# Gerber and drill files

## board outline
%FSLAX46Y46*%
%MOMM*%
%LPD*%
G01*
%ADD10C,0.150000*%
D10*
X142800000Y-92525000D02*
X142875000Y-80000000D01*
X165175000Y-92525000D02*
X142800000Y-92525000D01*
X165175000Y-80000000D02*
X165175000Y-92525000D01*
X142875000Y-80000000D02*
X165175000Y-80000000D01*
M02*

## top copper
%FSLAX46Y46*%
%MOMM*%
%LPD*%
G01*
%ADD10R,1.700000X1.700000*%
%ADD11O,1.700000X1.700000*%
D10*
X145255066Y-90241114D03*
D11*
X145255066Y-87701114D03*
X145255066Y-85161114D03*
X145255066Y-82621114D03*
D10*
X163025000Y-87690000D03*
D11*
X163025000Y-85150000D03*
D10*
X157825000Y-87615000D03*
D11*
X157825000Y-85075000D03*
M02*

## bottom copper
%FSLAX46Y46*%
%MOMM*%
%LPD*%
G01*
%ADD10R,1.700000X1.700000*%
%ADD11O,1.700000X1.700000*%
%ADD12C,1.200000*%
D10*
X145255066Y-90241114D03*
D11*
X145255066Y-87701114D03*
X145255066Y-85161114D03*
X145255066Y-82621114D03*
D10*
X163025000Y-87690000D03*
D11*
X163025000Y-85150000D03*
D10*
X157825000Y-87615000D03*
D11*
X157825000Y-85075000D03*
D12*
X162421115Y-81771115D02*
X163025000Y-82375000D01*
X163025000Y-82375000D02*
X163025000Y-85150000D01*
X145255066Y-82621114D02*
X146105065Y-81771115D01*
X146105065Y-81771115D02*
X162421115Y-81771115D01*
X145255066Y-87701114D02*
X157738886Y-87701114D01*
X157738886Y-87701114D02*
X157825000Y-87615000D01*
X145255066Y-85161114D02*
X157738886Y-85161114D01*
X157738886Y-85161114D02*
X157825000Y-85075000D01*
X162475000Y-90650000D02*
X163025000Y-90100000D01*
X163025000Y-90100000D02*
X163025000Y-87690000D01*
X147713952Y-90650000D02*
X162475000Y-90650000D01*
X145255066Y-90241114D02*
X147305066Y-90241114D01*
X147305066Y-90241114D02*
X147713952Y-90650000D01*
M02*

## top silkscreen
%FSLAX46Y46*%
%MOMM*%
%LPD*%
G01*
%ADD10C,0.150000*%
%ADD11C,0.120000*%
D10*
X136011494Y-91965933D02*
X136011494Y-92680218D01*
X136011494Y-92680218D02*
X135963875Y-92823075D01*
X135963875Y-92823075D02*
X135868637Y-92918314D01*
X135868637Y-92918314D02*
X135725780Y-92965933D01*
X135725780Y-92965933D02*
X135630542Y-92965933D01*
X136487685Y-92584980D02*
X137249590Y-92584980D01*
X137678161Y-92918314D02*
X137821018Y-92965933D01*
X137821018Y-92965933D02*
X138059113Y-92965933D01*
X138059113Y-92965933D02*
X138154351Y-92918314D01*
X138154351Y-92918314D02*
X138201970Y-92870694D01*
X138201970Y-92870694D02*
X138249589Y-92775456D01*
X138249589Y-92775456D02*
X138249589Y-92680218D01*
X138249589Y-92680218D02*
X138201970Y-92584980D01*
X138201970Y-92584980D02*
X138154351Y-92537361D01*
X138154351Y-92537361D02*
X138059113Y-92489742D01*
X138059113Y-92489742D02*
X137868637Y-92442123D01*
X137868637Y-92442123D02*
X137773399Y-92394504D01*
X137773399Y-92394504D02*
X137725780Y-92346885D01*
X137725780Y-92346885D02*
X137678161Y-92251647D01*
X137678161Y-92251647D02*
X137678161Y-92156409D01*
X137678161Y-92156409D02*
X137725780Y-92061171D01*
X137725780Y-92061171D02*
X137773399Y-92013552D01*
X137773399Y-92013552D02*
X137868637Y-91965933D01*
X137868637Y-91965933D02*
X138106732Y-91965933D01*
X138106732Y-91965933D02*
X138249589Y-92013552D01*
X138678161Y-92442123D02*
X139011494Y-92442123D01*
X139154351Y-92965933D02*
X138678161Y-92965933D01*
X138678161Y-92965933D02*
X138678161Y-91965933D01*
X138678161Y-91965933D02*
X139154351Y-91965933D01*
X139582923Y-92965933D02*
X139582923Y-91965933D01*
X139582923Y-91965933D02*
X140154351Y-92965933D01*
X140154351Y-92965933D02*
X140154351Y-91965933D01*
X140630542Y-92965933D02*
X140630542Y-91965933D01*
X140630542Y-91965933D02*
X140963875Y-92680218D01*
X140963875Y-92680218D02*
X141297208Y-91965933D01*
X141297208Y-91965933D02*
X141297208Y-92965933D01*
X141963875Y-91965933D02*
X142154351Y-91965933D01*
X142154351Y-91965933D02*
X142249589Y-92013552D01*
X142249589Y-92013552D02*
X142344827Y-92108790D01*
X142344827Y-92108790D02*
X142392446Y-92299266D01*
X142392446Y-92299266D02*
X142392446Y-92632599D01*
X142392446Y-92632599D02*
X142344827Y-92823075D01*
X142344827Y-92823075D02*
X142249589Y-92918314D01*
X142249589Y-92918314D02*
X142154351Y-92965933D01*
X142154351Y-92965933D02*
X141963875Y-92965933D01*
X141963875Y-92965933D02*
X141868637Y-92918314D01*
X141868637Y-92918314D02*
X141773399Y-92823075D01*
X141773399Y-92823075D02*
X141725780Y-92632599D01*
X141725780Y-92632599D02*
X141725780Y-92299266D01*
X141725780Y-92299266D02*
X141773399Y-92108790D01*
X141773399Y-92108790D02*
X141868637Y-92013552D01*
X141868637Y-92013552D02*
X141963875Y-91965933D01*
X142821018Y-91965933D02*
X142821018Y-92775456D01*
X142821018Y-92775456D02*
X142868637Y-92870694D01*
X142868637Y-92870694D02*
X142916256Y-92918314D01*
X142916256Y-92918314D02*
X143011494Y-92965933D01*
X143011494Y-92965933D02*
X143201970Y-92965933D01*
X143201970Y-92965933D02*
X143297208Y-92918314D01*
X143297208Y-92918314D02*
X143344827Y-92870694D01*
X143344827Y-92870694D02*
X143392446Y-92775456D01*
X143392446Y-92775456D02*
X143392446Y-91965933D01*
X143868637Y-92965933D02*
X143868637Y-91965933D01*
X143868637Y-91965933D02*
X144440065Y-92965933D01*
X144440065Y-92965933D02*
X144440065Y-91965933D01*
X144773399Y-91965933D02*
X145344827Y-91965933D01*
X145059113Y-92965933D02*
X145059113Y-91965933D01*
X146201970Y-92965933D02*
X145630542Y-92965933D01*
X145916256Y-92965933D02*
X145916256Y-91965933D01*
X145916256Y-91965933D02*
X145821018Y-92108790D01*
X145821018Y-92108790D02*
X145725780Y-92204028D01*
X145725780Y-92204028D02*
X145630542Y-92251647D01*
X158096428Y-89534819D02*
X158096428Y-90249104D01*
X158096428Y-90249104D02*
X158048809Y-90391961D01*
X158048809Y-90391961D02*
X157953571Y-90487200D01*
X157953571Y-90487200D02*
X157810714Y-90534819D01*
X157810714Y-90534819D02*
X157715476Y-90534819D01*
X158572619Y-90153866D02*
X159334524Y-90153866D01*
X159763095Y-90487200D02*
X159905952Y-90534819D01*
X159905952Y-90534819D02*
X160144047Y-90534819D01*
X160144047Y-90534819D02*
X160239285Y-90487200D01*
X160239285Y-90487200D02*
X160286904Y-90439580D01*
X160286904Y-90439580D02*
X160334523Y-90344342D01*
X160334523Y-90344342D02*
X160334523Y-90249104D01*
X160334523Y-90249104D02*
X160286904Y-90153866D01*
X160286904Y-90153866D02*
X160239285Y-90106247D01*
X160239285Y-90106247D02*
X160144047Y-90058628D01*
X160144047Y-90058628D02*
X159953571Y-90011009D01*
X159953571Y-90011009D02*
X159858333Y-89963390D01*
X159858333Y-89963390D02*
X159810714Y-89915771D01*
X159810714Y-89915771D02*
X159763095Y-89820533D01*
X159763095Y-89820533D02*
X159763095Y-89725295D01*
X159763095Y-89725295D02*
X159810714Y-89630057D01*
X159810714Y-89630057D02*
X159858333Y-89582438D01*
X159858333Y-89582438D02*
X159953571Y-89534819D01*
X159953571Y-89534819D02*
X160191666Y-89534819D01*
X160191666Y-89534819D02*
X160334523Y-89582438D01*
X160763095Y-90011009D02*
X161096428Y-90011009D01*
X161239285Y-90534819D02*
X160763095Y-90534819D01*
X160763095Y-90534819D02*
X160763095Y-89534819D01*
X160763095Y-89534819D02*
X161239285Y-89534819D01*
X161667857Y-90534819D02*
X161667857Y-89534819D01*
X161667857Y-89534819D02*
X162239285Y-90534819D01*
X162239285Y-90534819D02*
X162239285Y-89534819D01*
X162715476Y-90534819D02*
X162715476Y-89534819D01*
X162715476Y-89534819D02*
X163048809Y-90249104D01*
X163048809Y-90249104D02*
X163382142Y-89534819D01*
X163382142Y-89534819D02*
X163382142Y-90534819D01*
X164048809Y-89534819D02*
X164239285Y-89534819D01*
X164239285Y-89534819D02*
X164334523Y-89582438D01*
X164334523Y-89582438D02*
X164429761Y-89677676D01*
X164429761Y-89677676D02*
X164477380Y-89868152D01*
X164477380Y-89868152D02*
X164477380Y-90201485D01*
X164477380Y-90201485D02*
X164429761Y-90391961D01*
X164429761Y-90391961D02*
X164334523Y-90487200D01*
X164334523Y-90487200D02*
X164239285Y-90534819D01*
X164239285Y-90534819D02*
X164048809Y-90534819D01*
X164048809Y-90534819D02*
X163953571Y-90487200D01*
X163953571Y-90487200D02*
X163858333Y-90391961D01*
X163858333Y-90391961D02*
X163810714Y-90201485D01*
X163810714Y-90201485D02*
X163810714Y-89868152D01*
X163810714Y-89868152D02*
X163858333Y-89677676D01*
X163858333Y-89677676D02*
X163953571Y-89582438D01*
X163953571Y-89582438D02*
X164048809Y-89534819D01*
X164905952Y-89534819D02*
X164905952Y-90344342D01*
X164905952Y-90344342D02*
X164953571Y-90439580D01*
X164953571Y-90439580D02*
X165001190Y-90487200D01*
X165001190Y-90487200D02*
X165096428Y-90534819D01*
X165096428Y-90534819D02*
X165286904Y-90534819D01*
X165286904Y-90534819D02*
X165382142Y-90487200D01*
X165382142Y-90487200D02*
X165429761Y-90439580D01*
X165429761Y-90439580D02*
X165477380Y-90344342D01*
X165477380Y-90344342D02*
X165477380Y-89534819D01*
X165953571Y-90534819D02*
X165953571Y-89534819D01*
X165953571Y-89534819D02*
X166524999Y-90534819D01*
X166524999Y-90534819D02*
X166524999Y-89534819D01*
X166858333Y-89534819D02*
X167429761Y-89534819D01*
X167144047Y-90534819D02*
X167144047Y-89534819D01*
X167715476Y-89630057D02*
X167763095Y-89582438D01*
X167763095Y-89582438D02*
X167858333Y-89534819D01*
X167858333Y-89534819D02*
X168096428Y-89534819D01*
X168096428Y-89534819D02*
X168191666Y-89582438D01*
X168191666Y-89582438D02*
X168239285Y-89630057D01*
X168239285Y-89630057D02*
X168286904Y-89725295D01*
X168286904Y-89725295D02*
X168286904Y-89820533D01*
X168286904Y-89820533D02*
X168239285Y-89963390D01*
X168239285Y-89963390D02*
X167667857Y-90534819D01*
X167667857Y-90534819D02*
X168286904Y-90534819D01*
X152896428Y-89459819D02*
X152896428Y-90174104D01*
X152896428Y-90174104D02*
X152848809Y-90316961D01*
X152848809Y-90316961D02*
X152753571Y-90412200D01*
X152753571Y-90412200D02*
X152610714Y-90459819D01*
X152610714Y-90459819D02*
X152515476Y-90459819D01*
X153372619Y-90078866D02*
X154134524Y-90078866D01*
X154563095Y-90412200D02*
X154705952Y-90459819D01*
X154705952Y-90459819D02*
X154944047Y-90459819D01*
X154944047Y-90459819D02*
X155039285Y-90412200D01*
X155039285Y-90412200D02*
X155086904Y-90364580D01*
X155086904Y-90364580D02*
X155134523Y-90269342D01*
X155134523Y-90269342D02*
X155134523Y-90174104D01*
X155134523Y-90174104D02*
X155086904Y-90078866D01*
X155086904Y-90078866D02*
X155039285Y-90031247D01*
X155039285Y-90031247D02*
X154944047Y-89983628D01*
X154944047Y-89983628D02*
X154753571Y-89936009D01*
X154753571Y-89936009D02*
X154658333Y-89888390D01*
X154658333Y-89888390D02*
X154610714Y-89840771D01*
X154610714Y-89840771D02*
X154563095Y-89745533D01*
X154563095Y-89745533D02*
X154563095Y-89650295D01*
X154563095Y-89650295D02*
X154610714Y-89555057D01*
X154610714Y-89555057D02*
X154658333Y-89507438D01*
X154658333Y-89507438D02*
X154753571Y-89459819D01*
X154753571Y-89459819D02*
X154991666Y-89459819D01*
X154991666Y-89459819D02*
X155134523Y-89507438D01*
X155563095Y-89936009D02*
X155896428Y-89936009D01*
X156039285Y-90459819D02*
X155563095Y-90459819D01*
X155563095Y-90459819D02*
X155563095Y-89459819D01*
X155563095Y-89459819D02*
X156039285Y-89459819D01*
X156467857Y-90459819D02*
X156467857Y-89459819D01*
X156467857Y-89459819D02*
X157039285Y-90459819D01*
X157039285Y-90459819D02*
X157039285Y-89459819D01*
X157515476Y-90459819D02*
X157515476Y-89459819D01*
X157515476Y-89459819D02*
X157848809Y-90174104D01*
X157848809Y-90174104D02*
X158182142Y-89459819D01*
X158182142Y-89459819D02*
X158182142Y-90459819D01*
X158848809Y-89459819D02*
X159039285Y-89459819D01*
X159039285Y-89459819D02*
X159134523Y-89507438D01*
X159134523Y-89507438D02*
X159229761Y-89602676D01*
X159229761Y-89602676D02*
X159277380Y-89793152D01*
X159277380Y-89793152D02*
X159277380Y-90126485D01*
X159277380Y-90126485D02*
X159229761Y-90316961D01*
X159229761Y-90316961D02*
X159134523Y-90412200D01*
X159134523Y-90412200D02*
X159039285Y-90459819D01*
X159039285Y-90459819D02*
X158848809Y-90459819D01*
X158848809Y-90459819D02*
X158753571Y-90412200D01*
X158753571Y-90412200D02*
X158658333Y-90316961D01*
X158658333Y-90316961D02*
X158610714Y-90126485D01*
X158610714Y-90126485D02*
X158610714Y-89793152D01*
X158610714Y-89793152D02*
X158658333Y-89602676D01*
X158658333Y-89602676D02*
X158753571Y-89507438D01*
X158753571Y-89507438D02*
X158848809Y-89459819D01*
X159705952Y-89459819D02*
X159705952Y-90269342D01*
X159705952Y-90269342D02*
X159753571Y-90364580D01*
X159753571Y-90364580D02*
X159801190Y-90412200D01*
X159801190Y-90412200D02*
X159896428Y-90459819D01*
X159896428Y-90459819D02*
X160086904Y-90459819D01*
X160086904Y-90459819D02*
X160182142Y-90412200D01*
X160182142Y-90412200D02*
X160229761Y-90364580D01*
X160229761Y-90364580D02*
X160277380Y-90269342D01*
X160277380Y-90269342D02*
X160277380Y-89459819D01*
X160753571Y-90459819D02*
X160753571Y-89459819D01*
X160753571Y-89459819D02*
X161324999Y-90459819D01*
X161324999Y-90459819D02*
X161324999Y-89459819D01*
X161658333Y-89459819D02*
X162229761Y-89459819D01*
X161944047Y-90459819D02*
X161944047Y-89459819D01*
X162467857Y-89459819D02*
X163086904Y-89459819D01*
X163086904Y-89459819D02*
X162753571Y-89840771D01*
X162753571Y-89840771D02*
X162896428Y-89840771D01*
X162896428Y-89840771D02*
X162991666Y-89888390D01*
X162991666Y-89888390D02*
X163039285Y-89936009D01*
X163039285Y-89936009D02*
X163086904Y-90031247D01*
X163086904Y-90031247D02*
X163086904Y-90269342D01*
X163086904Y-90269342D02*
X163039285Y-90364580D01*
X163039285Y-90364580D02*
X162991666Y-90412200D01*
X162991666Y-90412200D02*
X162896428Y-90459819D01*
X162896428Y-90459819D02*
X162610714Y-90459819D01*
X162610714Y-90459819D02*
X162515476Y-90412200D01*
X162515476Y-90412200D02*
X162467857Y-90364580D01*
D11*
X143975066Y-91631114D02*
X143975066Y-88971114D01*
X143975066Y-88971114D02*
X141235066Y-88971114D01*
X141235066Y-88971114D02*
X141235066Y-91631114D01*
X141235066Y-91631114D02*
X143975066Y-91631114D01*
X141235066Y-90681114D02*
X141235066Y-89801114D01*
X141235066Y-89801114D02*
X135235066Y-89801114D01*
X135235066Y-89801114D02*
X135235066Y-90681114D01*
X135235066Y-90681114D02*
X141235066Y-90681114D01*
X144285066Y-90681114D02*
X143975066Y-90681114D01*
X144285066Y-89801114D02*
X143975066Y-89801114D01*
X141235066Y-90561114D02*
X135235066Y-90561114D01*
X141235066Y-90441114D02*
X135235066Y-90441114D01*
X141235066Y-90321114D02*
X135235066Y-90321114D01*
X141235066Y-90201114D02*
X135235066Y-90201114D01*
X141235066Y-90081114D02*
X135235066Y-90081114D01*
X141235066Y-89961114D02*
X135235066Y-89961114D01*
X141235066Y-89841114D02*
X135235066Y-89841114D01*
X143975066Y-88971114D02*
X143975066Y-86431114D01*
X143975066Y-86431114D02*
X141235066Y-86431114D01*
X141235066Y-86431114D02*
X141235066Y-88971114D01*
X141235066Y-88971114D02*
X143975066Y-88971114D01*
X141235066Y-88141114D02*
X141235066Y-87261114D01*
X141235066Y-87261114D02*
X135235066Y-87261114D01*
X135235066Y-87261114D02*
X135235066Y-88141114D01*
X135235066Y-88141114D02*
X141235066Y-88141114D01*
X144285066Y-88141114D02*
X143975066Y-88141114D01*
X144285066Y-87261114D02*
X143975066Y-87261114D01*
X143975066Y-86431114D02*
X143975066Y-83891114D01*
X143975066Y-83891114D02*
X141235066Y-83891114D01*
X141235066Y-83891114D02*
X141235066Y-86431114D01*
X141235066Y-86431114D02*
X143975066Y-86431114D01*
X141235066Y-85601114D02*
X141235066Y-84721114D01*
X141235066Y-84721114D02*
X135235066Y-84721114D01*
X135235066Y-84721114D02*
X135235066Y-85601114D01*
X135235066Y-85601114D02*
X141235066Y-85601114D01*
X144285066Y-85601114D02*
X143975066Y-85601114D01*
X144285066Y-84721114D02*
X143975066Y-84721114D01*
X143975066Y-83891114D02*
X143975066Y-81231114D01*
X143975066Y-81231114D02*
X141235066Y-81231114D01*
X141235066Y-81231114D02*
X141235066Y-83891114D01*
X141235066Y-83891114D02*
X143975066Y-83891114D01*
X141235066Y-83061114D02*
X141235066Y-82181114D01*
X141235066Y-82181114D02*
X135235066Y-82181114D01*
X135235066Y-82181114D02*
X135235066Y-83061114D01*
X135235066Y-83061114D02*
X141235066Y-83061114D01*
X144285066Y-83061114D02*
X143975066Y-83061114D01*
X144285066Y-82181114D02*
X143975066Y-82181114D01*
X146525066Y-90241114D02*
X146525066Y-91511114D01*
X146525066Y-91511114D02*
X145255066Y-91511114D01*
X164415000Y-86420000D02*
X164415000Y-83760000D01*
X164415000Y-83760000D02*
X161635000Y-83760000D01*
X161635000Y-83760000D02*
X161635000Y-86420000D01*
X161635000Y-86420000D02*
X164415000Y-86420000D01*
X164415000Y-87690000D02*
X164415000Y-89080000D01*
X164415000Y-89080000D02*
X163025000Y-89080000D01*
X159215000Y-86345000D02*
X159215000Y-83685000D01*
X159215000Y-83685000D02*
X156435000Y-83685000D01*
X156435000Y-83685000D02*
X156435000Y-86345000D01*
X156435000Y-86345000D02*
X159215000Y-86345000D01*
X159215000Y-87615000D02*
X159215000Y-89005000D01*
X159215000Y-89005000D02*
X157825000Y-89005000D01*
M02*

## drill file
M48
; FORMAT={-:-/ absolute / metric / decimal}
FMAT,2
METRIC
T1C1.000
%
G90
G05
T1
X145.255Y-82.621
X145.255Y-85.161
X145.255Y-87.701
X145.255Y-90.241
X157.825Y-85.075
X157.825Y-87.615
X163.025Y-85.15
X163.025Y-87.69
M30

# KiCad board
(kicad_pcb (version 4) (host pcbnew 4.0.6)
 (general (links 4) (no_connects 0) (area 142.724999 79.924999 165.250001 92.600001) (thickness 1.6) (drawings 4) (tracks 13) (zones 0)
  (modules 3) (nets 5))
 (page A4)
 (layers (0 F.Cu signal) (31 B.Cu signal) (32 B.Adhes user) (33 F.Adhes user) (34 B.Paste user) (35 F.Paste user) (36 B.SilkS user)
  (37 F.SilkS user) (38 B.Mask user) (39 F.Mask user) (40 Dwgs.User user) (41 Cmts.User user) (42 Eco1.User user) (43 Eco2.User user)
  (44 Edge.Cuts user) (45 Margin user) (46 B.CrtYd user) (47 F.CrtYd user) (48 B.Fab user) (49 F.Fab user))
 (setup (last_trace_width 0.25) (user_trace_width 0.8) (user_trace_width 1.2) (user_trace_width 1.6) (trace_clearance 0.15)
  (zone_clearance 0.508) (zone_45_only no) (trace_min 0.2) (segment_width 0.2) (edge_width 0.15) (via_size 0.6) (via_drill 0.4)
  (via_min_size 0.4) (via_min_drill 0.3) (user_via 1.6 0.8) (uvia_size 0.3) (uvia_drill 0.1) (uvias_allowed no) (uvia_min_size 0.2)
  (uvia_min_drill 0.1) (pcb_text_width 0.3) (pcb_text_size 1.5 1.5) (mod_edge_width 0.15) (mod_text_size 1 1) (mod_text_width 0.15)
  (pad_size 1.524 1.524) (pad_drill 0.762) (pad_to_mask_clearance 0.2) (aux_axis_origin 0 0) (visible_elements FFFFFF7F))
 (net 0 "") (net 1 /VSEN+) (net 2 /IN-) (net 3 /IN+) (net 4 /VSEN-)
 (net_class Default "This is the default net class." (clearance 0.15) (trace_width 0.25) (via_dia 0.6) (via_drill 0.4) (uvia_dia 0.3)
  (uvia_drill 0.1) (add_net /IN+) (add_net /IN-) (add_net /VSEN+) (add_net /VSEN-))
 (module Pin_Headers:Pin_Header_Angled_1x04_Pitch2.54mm (layer F.Cu) (at 145.255066 90.241114 180)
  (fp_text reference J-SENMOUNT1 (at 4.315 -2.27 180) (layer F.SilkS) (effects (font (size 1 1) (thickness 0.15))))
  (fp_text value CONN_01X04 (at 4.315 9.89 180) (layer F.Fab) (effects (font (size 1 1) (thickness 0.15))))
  (fp_line (start 1.28 -1.39) (end 1.28 1.27) (layer F.SilkS) (width 0.12))
  (fp_line (start 1.28 1.27) (end 4.02 1.27) (layer F.SilkS) (width 0.12))
  (fp_line (start 4.02 1.27) (end 4.02 -1.39) (layer F.SilkS) (width 0.12))
  (fp_line (start 4.02 -1.39) (end 1.28 -1.39) (layer F.SilkS) (width 0.12))
  (fp_line (start 4.02 -0.44) (end 4.02 0.44) (layer F.SilkS) (width 0.12))
  (fp_line (start 4.02 0.44) (end 10.02 0.44) (layer F.SilkS) (width 0.12))
  (fp_line (start 10.02 0.44) (end 10.02 -0.44) (layer F.SilkS) (width 0.12))
  (fp_line (start 10.02 -0.44) (end 4.02 -0.44) (layer F.SilkS) (width 0.12))
  (fp_line (start 0.97 -0.44) (end 1.28 -0.44) (layer F.SilkS) (width 0.12))
  (fp_line (start 0.97 0.44) (end 1.28 0.44) (layer F.SilkS) (width 0.12))
  (fp_line (start 4.02 -0.32) (end 10.02 -0.32) (layer F.SilkS) (width 0.12))
  (fp_line (start 4.02 -0.2) (end 10.02 -0.2) (layer F.SilkS) (width 0.12))
  (fp_line (start 4.02 -0.08) (end 10.02 -0.08) (layer F.SilkS) (width 0.12))
  (fp_line (start 4.02 0.04) (end 10.02 0.04) (layer F.SilkS) (width 0.12))
  (fp_line (start 4.02 0.16) (end 10.02 0.16) (layer F.SilkS) (width 0.12))
  (fp_line (start 4.02 0.28) (end 10.02 0.28) (layer F.SilkS) (width 0.12))
  (fp_line (start 4.02 0.4) (end 10.02 0.4) (layer F.SilkS) (width 0.12))
  (fp_line (start 1.28 1.27) (end 1.28 3.81) (layer F.SilkS) (width 0.12))
  (fp_line (start 1.28 3.81) (end 4.02 3.81) (layer F.SilkS) (width 0.12))
  (fp_line (start 4.02 3.81) (end 4.02 1.27) (layer F.SilkS) (width 0.12))
  (fp_line (start 4.02 1.27) (end 1.28 1.27) (layer F.SilkS) (width 0.12))
  (fp_line (start 4.02 2.1) (end 4.02 2.98) (layer F.SilkS) (width 0.12))
  (fp_line (start 4.02 2.98) (end 10.02 2.98) (layer F.SilkS) (width 0.12))
  (fp_line (start 10.02 2.98) (end 10.02 2.1) (layer F.SilkS) (width 0.12))
  (fp_line (start 10.02 2.1) (end 4.02 2.1) (layer F.SilkS) (width 0.12))
  (fp_line (start 0.97 2.1) (end 1.28 2.1) (layer F.SilkS) (width 0.12))
  (fp_line (start 0.97 2.98) (end 1.28 2.98) (layer F.SilkS) (width 0.12))
  (fp_line (start 1.28 3.81) (end 1.28 6.35) (layer F.SilkS) (width 0.12))
  (fp_line (start 1.28 6.35) (end 4.02 6.35) (layer F.SilkS) (width 0.12))
  (fp_line (start 4.02 6.35) (end 4.02 3.81) (layer F.SilkS) (width 0.12))
  (fp_line (start 4.02 3.81) (end 1.28 3.81) (layer F.SilkS) (width 0.12))
  (fp_line (start 4.02 4.64) (end 4.02 5.52) (layer F.SilkS) (width 0.12))
  (fp_line (start 4.02 5.52) (end 10.02 5.52) (layer F.SilkS) (width 0.12))
  (fp_line (start 10.02 5.52) (end 10.02 4.64) (layer F.SilkS) (width 0.12))
  (fp_line (start 10.02 4.64) (end 4.02 4.64) (layer F.SilkS) (width 0.12))
  (fp_line (start 0.97 4.64) (end 1.28 4.64) (layer F.SilkS) (width 0.12))
  (fp_line (start 0.97 5.52) (end 1.28 5.52) (layer F.SilkS) (width 0.12))
  (fp_line (start 1.28 6.35) (end 1.28 9.01) (layer F.SilkS) (width 0.12))
  (fp_line (start 1.28 9.01) (end 4.02 9.01) (layer F.SilkS) (width 0.12))
  (fp_line (start 4.02 9.01) (end 4.02 6.35) (layer F.SilkS) (width 0.12))
  (fp_line (start 4.02 6.35) (end 1.28 6.35) (layer F.SilkS) (width 0.12))
  (fp_line (start 4.02 7.18) (end 4.02 8.06) (layer F.SilkS) (width 0.12))
  (fp_line (start 4.02 8.06) (end 10.02 8.06) (layer F.SilkS) (width 0.12))
  (fp_line (start 10.02 8.06) (end 10.02 7.18) (layer F.SilkS) (width 0.12))
  (fp_line (start 10.02 7.18) (end 4.02 7.18) (layer F.SilkS) (width 0.12))
  (fp_line (start 0.97 7.18) (end 1.28 7.18) (layer F.SilkS) (width 0.12))
  (fp_line (start 0.97 8.06) (end 1.28 8.06) (layer F.SilkS) (width 0.12))
  (fp_line (start -1.27 0) (end -1.27 -1.27) (layer F.SilkS) (width 0.12))
  (fp_line (start -1.27 -1.27) (end 0 -1.27) (layer F.SilkS) (width 0.12))
  (pad 1 thru_hole rect (at 0 0 180) (size 1.7 1.7) (drill 1) (layers *.Cu *.Mask) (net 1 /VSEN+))
  (pad 2 thru_hole oval (at 0 2.54 180) (size 1.7 1.7) (drill 1) (layers *.Cu *.Mask) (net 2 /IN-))
  (pad 3 thru_hole oval (at 0 5.08 180) (size 1.7 1.7) (drill 1) (layers *.Cu *.Mask) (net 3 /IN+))
  (pad 4 thru_hole oval (at 0 7.62 180) (size 1.7 1.7) (drill 1) (layers *.Cu *.Mask) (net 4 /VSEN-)))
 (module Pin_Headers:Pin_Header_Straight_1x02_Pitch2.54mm (layer F.Cu) (at 163.025 87.69 180)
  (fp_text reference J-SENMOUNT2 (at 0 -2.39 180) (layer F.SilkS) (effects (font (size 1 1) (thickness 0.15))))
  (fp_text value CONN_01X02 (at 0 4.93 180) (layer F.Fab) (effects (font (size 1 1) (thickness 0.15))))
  (fp_line (start -1.39 1.27) (end -1.39 3.93) (layer F.SilkS) (width 0.12))
  (fp_line (start -1.39 3.93) (end 1.39 3.93) (layer F.SilkS) (width 0.12))
  (fp_line (start 1.39 3.93) (end 1.39 1.27) (layer F.SilkS) (width 0.12))
  (fp_line (start 1.39 1.27) (end -1.39 1.27) (layer F.SilkS) (width 0.12))
  (fp_line (start -1.39 0) (end -1.39 -1.39) (layer F.SilkS) (width 0.12))
  (fp_line (start -1.39 -1.39) (end 0 -1.39) (layer F.SilkS) (width 0.12))
  (pad 1 thru_hole rect (at 0 0 180) (size 1.7 1.7) (drill 1) (layers *.Cu *.Mask) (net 1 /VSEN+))
  (pad 2 thru_hole oval (at 0 2.54 180) (size 1.7 1.7) (drill 1) (layers *.Cu *.Mask) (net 4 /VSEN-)))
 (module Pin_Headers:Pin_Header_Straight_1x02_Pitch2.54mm (layer F.Cu) (at 157.825 87.615 180)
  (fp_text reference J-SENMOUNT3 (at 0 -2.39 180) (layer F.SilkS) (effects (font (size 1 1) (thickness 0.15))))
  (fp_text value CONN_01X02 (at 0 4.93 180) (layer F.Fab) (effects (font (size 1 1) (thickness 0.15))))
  (fp_line (start -1.39 1.27) (end -1.39 3.93) (layer F.SilkS) (width 0.12))
  (fp_line (start -1.39 3.93) (end 1.39 3.93) (layer F.SilkS) (width 0.12))
  (fp_line (start 1.39 3.93) (end 1.39 1.27) (layer F.SilkS) (width 0.12))
  (fp_line (start 1.39 1.27) (end -1.39 1.27) (layer F.SilkS) (width 0.12))
  (fp_line (start -1.39 0) (end -1.39 -1.39) (layer F.SilkS) (width 0.12))
  (fp_line (start -1.39 -1.39) (end 0 -1.39) (layer F.SilkS) (width 0.12))
  (pad 1 thru_hole rect (at 0 0 180) (size 1.7 1.7) (drill 1) (layers *.Cu *.Mask) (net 2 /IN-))
  (pad 2 thru_hole oval (at 0 2.54 180) (size 1.7 1.7) (drill 1) (layers *.Cu *.Mask) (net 3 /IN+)))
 (gr_line (start 142.8 92.525) (end 142.875 80) (layer Edge.Cuts) (width 0.15))
 (gr_line (start 165.175 92.525) (end 142.8 92.525) (layer Edge.Cuts) (width 0.15))
 (gr_line (start 165.175 80) (end 165.175 92.525) (layer Edge.Cuts) (width 0.15))
 (gr_line (start 142.875 80) (end 165.175 80) (layer Edge.Cuts) (width 0.15))
 (segment (start 162.421115 81.771115) (end 163.025 82.375) (width 1.2) (layer B.Cu) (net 4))
 (segment (start 163.025 82.375) (end 163.025 85.15) (width 1.2) (layer B.Cu) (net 4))
 (segment (start 145.255066 82.621114) (end 146.105065 81.771115) (width 1.2) (layer B.Cu) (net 4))
 (segment (start 146.105065 81.771115) (end 162.421115 81.771115) (width 1.2) (layer B.Cu) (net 4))
 (segment (start 145.255066 87.701114) (end 157.738886 87.701114) (width 1.2) (layer B.Cu) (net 2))
 (segment (start 157.738886 87.701114) (end 157.825 87.615) (width 1.2) (layer B.Cu) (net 2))
 (segment (start 145.255066 85.161114) (end 157.738886 85.161114) (width 1.2) (layer B.Cu) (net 3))
 (segment (start 157.738886 85.161114) (end 157.825 85.075) (width 1.2) (layer B.Cu) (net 3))
 (segment (start 162.475 90.65) (end 163.025 90.1) (width 1.2) (layer B.Cu) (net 1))
 (segment (start 163.025 90.1) (end 163.025 87.69) (width 1.2) (layer B.Cu) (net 1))
 (segment (start 147.713952 90.65) (end 162.475 90.65) (width 1.2) (layer B.Cu) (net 1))
 (segment (start 145.255066 90.241114) (end 147.305066 90.241114) (width 1.2) (layer B.Cu) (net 1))
 (segment (start 147.305066 90.241114) (end 147.713952 90.65) (width 1.2) (layer B.Cu) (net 1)))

